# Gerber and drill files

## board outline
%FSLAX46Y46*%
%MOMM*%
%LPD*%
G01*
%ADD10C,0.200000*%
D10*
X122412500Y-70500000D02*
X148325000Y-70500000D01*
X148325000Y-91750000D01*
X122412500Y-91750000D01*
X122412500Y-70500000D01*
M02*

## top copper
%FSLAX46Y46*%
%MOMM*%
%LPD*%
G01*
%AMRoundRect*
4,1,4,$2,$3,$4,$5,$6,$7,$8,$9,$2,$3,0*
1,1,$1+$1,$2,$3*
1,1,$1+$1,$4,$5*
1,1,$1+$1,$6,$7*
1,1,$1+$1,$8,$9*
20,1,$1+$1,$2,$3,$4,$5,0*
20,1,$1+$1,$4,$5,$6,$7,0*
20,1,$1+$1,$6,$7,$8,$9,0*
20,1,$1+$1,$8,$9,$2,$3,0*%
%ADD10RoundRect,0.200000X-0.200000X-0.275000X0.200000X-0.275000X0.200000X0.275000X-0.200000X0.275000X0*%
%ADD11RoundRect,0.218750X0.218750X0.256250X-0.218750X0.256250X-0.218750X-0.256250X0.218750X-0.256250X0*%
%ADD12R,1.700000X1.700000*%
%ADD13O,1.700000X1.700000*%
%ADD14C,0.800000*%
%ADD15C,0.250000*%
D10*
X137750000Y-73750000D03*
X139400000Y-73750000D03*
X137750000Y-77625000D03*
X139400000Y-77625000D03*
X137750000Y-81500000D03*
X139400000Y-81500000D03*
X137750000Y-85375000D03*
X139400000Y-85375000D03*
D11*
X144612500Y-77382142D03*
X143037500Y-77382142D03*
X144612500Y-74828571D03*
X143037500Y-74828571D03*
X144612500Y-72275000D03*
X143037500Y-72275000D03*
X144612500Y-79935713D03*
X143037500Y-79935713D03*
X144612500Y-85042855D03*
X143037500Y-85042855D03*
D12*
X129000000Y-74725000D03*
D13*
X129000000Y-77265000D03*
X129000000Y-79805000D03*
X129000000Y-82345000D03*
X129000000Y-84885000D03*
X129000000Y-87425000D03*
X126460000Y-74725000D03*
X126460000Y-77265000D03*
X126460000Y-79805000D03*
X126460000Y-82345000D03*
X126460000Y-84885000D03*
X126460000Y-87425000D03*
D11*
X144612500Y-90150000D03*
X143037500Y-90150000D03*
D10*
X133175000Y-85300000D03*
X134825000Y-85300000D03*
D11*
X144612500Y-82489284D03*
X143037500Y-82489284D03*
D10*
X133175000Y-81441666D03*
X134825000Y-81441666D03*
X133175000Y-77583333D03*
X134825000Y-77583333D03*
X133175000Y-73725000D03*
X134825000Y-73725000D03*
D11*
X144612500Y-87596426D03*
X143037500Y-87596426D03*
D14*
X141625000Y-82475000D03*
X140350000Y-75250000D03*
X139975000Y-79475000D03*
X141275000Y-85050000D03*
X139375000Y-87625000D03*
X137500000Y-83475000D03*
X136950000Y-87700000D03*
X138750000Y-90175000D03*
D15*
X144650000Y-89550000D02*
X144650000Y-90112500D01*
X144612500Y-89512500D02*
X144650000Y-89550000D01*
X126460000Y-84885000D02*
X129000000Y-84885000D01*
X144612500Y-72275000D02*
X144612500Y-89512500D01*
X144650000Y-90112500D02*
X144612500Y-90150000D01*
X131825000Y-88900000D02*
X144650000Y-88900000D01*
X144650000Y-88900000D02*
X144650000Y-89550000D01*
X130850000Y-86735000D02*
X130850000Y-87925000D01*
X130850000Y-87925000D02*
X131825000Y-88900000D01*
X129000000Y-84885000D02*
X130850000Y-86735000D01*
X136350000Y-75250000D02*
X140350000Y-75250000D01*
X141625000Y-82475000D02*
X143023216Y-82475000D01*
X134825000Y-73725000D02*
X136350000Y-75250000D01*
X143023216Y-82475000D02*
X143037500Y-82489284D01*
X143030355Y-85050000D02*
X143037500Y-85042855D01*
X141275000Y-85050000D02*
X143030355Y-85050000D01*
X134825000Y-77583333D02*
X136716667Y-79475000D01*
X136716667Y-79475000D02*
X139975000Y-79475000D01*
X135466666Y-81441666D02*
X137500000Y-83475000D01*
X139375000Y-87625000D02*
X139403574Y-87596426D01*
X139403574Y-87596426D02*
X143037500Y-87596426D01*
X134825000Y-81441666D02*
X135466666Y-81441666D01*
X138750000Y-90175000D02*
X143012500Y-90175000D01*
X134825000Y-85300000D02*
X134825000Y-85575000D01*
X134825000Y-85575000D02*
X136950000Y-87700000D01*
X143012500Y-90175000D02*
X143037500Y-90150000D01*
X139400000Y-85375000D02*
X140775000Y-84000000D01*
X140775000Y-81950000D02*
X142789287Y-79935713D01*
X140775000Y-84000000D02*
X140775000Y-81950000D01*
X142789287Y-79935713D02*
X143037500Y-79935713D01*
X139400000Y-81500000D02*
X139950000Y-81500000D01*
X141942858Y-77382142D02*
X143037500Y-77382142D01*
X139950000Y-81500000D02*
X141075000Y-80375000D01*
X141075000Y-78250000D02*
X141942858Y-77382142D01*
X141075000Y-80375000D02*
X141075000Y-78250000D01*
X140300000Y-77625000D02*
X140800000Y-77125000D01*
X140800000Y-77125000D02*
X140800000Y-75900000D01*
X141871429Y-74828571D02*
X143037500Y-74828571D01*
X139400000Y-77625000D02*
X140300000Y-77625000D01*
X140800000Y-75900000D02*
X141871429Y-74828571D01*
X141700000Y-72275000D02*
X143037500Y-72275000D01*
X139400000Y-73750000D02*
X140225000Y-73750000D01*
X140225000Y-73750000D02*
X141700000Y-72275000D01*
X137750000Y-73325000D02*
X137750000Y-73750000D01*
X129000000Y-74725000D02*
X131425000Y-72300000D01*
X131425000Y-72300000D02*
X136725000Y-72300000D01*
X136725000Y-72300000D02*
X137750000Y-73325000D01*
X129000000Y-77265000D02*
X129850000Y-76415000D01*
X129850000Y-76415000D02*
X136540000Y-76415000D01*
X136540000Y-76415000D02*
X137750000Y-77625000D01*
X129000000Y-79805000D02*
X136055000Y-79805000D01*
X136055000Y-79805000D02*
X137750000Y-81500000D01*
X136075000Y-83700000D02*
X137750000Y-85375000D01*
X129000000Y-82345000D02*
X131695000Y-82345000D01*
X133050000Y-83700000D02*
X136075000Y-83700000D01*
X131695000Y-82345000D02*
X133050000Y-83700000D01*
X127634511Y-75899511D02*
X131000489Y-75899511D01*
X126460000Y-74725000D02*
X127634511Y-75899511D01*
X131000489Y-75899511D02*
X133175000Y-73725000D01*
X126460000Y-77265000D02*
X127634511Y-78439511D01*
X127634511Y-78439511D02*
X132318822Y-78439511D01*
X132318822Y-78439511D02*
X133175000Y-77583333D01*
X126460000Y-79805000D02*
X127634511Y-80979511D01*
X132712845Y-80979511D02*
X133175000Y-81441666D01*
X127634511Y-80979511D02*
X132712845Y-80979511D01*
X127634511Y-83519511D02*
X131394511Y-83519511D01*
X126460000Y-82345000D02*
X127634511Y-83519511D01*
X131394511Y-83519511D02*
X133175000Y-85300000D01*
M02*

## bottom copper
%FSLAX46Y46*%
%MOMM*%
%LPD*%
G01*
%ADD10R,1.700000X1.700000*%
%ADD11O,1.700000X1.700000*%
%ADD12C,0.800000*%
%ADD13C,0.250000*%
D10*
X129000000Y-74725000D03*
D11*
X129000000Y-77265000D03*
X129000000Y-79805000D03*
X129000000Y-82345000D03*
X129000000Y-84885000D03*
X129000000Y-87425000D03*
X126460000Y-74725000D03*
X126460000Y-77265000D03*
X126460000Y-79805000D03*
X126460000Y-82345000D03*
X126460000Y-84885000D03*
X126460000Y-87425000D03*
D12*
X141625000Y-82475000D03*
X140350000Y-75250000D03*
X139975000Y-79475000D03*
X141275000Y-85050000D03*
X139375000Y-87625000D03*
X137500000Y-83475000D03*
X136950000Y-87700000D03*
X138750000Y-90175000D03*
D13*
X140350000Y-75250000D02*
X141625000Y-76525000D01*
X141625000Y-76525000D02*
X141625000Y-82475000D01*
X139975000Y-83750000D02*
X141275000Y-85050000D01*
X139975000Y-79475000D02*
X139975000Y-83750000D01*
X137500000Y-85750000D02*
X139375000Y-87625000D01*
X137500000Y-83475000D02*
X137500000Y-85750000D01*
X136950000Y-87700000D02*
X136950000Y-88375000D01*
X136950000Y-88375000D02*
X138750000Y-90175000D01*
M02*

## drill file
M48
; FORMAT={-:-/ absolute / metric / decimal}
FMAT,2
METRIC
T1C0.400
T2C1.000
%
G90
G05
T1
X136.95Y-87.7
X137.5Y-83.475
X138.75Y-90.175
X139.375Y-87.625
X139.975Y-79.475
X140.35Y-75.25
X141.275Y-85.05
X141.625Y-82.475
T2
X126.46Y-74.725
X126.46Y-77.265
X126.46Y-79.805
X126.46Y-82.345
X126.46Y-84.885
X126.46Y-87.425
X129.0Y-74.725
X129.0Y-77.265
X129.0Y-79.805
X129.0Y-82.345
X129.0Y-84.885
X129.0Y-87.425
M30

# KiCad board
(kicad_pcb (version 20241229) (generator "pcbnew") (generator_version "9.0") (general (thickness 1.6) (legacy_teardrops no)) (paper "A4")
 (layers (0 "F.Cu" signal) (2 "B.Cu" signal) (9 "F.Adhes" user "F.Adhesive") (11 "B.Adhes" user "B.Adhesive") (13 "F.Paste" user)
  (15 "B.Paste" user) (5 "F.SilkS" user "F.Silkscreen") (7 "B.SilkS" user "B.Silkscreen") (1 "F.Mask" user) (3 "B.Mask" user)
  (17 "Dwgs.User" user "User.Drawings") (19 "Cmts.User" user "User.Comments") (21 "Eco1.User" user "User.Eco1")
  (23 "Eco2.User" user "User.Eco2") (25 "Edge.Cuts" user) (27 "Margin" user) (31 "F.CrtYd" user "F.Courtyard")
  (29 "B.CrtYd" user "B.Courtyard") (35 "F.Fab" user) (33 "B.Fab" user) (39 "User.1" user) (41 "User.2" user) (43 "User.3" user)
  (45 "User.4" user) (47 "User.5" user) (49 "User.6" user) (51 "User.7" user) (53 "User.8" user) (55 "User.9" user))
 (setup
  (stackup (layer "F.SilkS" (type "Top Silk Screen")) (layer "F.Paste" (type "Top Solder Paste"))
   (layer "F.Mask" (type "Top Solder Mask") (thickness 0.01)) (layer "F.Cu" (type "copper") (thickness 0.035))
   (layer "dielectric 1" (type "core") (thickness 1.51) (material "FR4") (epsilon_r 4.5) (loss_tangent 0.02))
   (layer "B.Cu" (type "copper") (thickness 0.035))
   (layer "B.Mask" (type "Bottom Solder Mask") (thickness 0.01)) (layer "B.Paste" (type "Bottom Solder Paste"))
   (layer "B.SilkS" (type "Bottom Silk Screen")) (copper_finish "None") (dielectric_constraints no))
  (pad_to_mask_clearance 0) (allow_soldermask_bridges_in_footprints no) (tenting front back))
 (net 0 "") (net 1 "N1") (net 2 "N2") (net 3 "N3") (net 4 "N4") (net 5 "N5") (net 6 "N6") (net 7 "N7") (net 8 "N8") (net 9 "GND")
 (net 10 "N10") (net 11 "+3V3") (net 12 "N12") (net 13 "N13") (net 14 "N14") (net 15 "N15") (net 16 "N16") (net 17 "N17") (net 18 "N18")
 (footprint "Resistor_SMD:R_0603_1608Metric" (layer "F.Cu") (at 138.575 73.75)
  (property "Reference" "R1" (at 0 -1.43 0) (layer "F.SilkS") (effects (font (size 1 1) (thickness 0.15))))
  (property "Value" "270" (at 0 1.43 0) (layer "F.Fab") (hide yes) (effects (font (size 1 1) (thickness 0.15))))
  (pad "1" smd roundrect (at -0.825 0) (size 0.8 0.95) (layers "F.Cu" "F.Mask" "F.Paste") (roundrect_rratio 0.25) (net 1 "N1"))
  (pad "2" smd roundrect (at 0.825 0) (size 0.8 0.95) (layers "F.Cu" "F.Mask" "F.Paste") (roundrect_rratio 0.25) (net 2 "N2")))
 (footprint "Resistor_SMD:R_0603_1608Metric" (layer "F.Cu") (at 138.575 77.625)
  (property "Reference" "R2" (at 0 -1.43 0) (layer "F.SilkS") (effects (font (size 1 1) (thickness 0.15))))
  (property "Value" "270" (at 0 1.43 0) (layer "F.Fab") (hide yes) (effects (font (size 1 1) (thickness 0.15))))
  (pad "1" smd roundrect (at -0.825 0) (size 0.8 0.95) (layers "F.Cu" "F.Mask" "F.Paste") (roundrect_rratio 0.25) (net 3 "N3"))
  (pad "2" smd roundrect (at 0.825 0) (size 0.8 0.95) (layers "F.Cu" "F.Mask" "F.Paste") (roundrect_rratio 0.25) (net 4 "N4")))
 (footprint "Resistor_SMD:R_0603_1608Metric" (layer "F.Cu") (at 138.575 81.5)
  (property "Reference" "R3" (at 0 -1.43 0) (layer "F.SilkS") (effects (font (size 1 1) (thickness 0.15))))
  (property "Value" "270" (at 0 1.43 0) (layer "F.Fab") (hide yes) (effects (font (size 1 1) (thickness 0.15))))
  (pad "1" smd roundrect (at -0.825 0) (size 0.8 0.95) (layers "F.Cu" "F.Mask" "F.Paste") (roundrect_rratio 0.25) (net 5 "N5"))
  (pad "2" smd roundrect (at 0.825 0) (size 0.8 0.95) (layers "F.Cu" "F.Mask" "F.Paste") (roundrect_rratio 0.25) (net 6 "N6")))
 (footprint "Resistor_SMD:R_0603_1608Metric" (layer "F.Cu") (at 138.575 85.375)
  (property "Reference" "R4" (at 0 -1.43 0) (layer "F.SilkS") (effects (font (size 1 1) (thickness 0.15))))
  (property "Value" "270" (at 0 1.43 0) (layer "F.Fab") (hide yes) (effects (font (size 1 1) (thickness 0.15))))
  (pad "1" smd roundrect (at -0.825 0) (size 0.8 0.95) (layers "F.Cu" "F.Mask" "F.Paste") (roundrect_rratio 0.25) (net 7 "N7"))
  (pad "2" smd roundrect (at 0.825 0) (size 0.8 0.95) (layers "F.Cu" "F.Mask" "F.Paste") (roundrect_rratio 0.25) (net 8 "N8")))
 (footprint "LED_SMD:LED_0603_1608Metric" (layer "F.Cu") (at 143.825 77.382142 180)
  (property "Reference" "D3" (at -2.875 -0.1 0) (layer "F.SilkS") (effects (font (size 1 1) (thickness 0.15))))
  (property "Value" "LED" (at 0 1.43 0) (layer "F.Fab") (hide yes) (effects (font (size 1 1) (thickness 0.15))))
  (pad "1" smd roundrect (at -0.7875 0 180) (size 0.875 0.95) (layers "F.Cu" "F.Mask" "F.Paste") (roundrect_rratio 0.25) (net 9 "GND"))
  (pad "2" smd roundrect (at 0.7875 0 180) (size 0.875 0.95) (layers "F.Cu" "F.Mask" "F.Paste") (roundrect_rratio 0.25) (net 6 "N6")))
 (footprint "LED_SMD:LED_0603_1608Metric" (layer "F.Cu") (at 143.825 74.828571 180)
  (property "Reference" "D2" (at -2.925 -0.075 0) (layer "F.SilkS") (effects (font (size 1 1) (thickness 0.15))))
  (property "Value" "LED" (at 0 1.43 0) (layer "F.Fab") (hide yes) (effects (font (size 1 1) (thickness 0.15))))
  (pad "1" smd roundrect (at -0.7875 0 180) (size 0.875 0.95) (layers "F.Cu" "F.Mask" "F.Paste") (roundrect_rratio 0.25) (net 9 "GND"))
  (pad "2" smd roundrect (at 0.7875 0 180) (size 0.875 0.95) (layers "F.Cu" "F.Mask" "F.Paste") (roundrect_rratio 0.25) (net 4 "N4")))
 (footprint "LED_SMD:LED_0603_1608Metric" (layer "F.Cu") (at 143.825 72.275 180)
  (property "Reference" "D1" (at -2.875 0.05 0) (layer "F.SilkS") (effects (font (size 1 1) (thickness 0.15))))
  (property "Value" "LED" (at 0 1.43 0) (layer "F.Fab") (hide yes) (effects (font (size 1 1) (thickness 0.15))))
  (pad "1" smd roundrect (at -0.7875 0 180) (size 0.875 0.95) (layers "F.Cu" "F.Mask" "F.Paste") (roundrect_rratio 0.25) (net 9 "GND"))
  (pad "2" smd roundrect (at 0.7875 0 180) (size 0.875 0.95) (layers "F.Cu" "F.Mask" "F.Paste") (roundrect_rratio 0.25) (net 2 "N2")))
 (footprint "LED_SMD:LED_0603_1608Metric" (layer "F.Cu") (at 143.825 79.935713 180)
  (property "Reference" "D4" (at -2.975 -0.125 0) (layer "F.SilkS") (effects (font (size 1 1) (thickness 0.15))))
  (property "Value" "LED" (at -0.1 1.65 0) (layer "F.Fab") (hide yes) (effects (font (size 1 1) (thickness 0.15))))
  (pad "1" smd roundrect (at -0.7875 0 180) (size 0.875 0.95) (layers "F.Cu" "F.Mask" "F.Paste") (roundrect_rratio 0.25) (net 9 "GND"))
  (pad "2" smd roundrect (at 0.7875 0 180) (size 0.875 0.95) (layers "F.Cu" "F.Mask" "F.Paste") (roundrect_rratio 0.25) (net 8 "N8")))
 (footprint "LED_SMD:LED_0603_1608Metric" (layer "F.Cu") (at 143.825 85.042855 180)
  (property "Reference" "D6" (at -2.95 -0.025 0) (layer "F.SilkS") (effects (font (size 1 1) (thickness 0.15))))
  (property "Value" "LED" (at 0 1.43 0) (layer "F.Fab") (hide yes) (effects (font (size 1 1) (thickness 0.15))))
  (pad "1" smd roundrect (at -0.7875 0 180) (size 0.875 0.95) (layers "F.Cu" "F.Mask" "F.Paste") (roundrect_rratio 0.25) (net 9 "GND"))
  (pad "2" smd roundrect (at 0.7875 0 180) (size 0.875 0.95) (layers "F.Cu" "F.Mask" "F.Paste") (roundrect_rratio 0.25) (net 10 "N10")))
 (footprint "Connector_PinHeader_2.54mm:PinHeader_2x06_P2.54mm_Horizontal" (layer "F.Cu") (at 129 87.425 180)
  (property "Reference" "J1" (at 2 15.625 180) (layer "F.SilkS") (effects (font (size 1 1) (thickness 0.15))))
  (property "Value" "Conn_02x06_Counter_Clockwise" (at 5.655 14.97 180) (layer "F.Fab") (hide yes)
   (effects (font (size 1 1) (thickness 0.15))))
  (pad "1" thru_hole rect (at 0 12.7 180) (size 1.7 1.7) (drill 1) (layers "*.Cu" "*.Mask") (remove_unused_layers no) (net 1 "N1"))
  (pad "2" thru_hole oval (at 0 10.16 180) (size 1.7 1.7) (drill 1) (layers "*.Cu" "*.Mask") (remove_unused_layers no) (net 3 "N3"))
  (pad "3" thru_hole oval (at 0 7.62 180) (size 1.7 1.7) (drill 1) (layers "*.Cu" "*.Mask") (remove_unused_layers no) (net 5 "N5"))
  (pad "4" thru_hole oval (at 0 5.08 180) (size 1.7 1.7) (drill 1) (layers "*.Cu" "*.Mask") (remove_unused_layers no) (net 7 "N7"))
  (pad "5" thru_hole oval (at 0 2.54 180) (size 1.7 1.7) (drill 1) (layers "*.Cu" "*.Mask") (remove_unused_layers no) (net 9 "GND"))
  (pad "6" thru_hole oval (at 0 0 180) (size 1.7 1.7) (drill 1) (layers "*.Cu" "*.Mask") (remove_unused_layers no) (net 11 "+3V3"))
  (pad "7" thru_hole oval (at 2.54 12.7 180) (size 1.7 1.7) (drill 1) (layers "*.Cu" "*.Mask") (remove_unused_layers no) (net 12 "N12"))
  (pad "8" thru_hole oval (at 2.54 10.16 180) (size 1.7 1.7) (drill 1) (layers "*.Cu" "*.Mask") (remove_unused_layers no) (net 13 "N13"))
  (pad "9" thru_hole oval (at 2.54 7.62 180) (size 1.7 1.7) (drill 1) (layers "*.Cu" "*.Mask") (remove_unused_layers no) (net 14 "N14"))
  (pad "10" thru_hole oval (at 2.54 5.08 180) (size 1.7 1.7) (drill 1) (layers "*.Cu" "*.Mask") (remove_unused_layers no) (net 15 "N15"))
  (pad "11" thru_hole oval (at 2.54 2.54 180) (size 1.7 1.7) (drill 1) (layers "*.Cu" "*.Mask") (remove_unused_layers no) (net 9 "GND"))
  (pad "12" thru_hole oval (at 2.54 0 180) (size 1.7 1.7) (drill 1) (layers "*.Cu" "*.Mask") (remove_unused_layers no) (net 11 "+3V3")))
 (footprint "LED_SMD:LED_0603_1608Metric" (layer "F.Cu") (at 143.825 90.15 180)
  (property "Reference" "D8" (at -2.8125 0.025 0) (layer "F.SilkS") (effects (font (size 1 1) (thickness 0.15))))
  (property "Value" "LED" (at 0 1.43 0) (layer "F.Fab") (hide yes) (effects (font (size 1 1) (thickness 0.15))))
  (pad "1" smd roundrect (at -0.7875 0 180) (size 0.875 0.95) (layers "F.Cu" "F.Mask" "F.Paste") (roundrect_rratio 0.25) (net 9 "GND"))
  (pad "2" smd roundrect (at 0.7875 0 180) (size 0.875 0.95) (layers "F.Cu" "F.Mask" "F.Paste") (roundrect_rratio 0.25) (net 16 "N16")))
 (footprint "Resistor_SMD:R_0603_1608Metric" (layer "F.Cu") (at 134 85.3)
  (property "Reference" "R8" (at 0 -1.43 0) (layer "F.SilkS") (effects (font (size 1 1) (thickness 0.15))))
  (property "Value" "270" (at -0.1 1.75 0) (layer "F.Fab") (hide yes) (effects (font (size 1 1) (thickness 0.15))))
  (pad "1" smd roundrect (at -0.825 0) (size 0.8 0.95) (layers "F.Cu" "F.Mask" "F.Paste") (roundrect_rratio 0.25) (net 15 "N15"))
  (pad "2" smd roundrect (at 0.825 0) (size 0.8 0.95) (layers "F.Cu" "F.Mask" "F.Paste") (roundrect_rratio 0.25) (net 16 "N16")))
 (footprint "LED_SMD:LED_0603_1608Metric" (layer "F.Cu") (at 143.825 82.489284 180)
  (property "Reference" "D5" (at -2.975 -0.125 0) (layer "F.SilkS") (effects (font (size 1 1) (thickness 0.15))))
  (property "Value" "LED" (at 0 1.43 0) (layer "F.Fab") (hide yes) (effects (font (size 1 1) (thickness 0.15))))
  (pad "1" smd roundrect (at -0.7875 0 180) (size 0.875 0.95) (layers "F.Cu" "F.Mask" "F.Paste") (roundrect_rratio 0.25) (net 9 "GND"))
  (pad "2" smd roundrect (at 0.7875 0 180) (size 0.875 0.95) (layers "F.Cu" "F.Mask" "F.Paste") (roundrect_rratio 0.25) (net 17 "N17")))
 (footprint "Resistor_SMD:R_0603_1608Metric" (layer "F.Cu") (at 134 81.441666)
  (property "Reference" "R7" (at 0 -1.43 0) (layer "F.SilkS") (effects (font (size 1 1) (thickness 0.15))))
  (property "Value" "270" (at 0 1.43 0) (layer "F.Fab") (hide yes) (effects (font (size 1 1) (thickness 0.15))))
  (pad "1" smd roundrect (at -0.825 0) (size 0.8 0.95) (layers "F.Cu" "F.Mask" "F.Paste") (roundrect_rratio 0.25) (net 14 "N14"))
  (pad "2" smd roundrect (at 0.825 0) (size 0.8 0.95) (layers "F.Cu" "F.Mask" "F.Paste") (roundrect_rratio 0.25) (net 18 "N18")))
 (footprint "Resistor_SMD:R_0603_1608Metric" (layer "F.Cu") (at 134 77.583333)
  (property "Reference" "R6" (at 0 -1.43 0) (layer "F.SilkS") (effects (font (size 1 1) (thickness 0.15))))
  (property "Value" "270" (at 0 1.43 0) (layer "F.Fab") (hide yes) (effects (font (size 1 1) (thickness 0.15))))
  (pad "1" smd roundrect (at -0.825 0) (size 0.8 0.95) (layers "F.Cu" "F.Mask" "F.Paste") (roundrect_rratio 0.25) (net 13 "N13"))
  (pad "2" smd roundrect (at 0.825 0) (size 0.8 0.95) (layers "F.Cu" "F.Mask" "F.Paste") (roundrect_rratio 0.25) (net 10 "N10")))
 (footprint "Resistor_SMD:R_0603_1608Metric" (layer "F.Cu") (at 134 73.725)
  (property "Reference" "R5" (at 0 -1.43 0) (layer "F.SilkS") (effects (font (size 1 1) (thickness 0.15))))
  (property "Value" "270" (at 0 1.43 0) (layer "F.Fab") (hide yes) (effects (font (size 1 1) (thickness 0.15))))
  (pad "1" smd roundrect (at -0.825 0) (size 0.8 0.95) (layers "F.Cu" "F.Mask" "F.Paste") (roundrect_rratio 0.25) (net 12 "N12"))
  (pad "2" smd roundrect (at 0.825 0) (size 0.8 0.95) (layers "F.Cu" "F.Mask" "F.Paste") (roundrect_rratio 0.25) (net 17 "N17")))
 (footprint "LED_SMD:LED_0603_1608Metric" (layer "F.Cu") (at 143.825 87.596426 180)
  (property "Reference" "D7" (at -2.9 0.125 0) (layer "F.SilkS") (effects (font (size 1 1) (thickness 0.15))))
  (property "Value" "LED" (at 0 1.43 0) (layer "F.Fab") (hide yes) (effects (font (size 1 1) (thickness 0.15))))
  (pad "1" smd roundrect (at -0.7875 0 180) (size 0.875 0.95) (layers "F.Cu" "F.Mask" "F.Paste") (roundrect_rratio 0.25) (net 9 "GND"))
  (pad "2" smd roundrect (at 0.7875 0 180) (size 0.875 0.95) (layers "F.Cu" "F.Mask" "F.Paste") (roundrect_rratio 0.25) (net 18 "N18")))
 (gr_rect (start 122.4125 70.5) (end 148.325 91.75) (stroke (width 0.2) (type solid)) (fill no) (layer "Edge.Cuts"))
 (segment (start 144.65 89.55) (end 144.65 90.1125) (width 0.25) (layer "F.Cu") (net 9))
 (segment (start 144.6125 89.5125) (end 144.65 89.55) (width 0.25) (layer "F.Cu") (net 9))
 (segment (start 126.46 84.885) (end 129 84.885) (width 0.25) (layer "F.Cu") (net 9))
 (segment (start 144.6125 72.275) (end 144.6125 89.5125) (width 0.25) (layer "F.Cu") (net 9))
 (segment (start 144.65 90.1125) (end 144.6125 90.15) (width 0.25) (layer "F.Cu") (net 9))
 (segment (start 131.825 88.9) (end 144.65 88.9) (width 0.25) (layer "F.Cu") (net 9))
 (segment (start 144.65 88.9) (end 144.65 89.55) (width 0.25) (layer "F.Cu") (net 9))
 (segment (start 130.85 86.735) (end 130.85 87.925) (width 0.25) (layer "F.Cu") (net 9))
 (segment (start 130.85 87.925) (end 131.825 88.9) (width 0.25) (layer "F.Cu") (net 9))
 (segment (start 129 84.885) (end 130.85 86.735) (width 0.25) (layer "F.Cu") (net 9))
 (segment (start 136.35 75.25) (end 140.35 75.25) (width 0.25) (layer "F.Cu") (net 17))
 (segment (start 141.625 82.475) (end 143.023216 82.475) (width 0.25) (layer "F.Cu") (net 17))
 (segment (start 134.825 73.725) (end 136.35 75.25) (width 0.25) (layer "F.Cu") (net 17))
 (segment (start 143.023216 82.475) (end 143.0375 82.489284) (width 0.25) (layer "F.Cu") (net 17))
 (via (at 141.625 82.475) (size 0.8) (drill 0.4) (layers "F.Cu" "B.Cu") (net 17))
 (via (at 140.35 75.25) (size 0.8) (drill 0.4) (layers "F.Cu" "B.Cu") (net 17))
 (segment (start 140.35 75.25) (end 141.625 76.525) (width 0.25) (layer "B.Cu") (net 17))
 (segment (start 141.625 76.525) (end 141.625 82.475) (width 0.25) (layer "B.Cu") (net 17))
 (segment (start 143.030355 85.05) (end 143.0375 85.042855) (width 0.25) (layer "F.Cu") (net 10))
 (segment (start 141.275 85.05) (end 143.030355 85.05) (width 0.25) (layer "F.Cu") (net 10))
 (segment (start 134.825 77.583333) (end 136.716667 79.475) (width 0.25) (layer "F.Cu") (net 10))
 (segment (start 136.716667 79.475) (end 139.975 79.475) (width 0.25) (layer "F.Cu") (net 10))
 (via (at 139.975 79.475) (size 0.8) (drill 0.4) (layers "F.Cu" "B.Cu") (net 10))
 (via (at 141.275 85.05) (size 0.8) (drill 0.4) (layers "F.Cu" "B.Cu") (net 10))
 (segment (start 139.975 83.75) (end 141.275 85.05) (width 0.25) (layer "B.Cu") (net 10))
 (segment (start 139.975 79.475) (end 139.975 83.75) (width 0.25) (layer "B.Cu") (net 10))
 (segment (start 135.466666 81.441666) (end 137.5 83.475) (width 0.25) (layer "F.Cu") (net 18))
 (segment (start 139.375 87.625) (end 139.403574 87.596426) (width 0.25) (layer "F.Cu") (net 18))
 (segment (start 139.403574 87.596426) (end 143.0375 87.596426) (width 0.25) (layer "F.Cu") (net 18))
 (segment (start 134.825 81.441666) (end 135.466666 81.441666) (width 0.25) (layer "F.Cu") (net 18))
 (via (at 139.375 87.625) (size 0.8) (drill 0.4) (layers "F.Cu" "B.Cu") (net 18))
 (via (at 137.5 83.475) (size 0.8) (drill 0.4) (layers "F.Cu" "B.Cu") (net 18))
 (segment (start 137.5 85.75) (end 139.375 87.625) (width 0.25) (layer "B.Cu") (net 18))
 (segment (start 137.5 83.475) (end 137.5 85.75) (width 0.25) (layer "B.Cu") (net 18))
 (segment (start 138.75 90.175) (end 143.0125 90.175) (width 0.25) (layer "F.Cu") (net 16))
 (segment (start 134.825 85.3) (end 134.825 85.575) (width 0.25) (layer "F.Cu") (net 16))
 (segment (start 134.825 85.575) (end 136.95 87.7) (width 0.25) (layer "F.Cu") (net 16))
 (segment (start 143.0125 90.175) (end 143.0375 90.15) (width 0.25) (layer "F.Cu") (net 16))
 (via (at 136.95 87.7) (size 0.8) (drill 0.4) (layers "F.Cu" "B.Cu") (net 16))
 (via (at 138.75 90.175) (size 0.8) (drill 0.4) (layers "F.Cu" "B.Cu") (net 16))
 (segment (start 136.95 87.7) (end 136.95 88.375) (width 0.25) (layer "B.Cu") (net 16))
 (segment (start 136.95 88.375) (end 138.75 90.175) (width 0.25) (layer "B.Cu") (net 16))
 (segment (start 139.4 85.375) (end 140.775 84) (width 0.25) (layer "F.Cu") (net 8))
 (segment (start 140.775 81.95) (end 142.789287 79.935713) (width 0.25) (layer "F.Cu") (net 8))
 (segment (start 140.775 84) (end 140.775 81.95) (width 0.25) (layer "F.Cu") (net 8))
 (segment (start 142.789287 79.935713) (end 143.0375 79.935713) (width 0.25) (layer "F.Cu") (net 8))
 (segment (start 139.4 81.5) (end 139.95 81.5) (width 0.25) (layer "F.Cu") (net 6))
 (segment (start 141.942858 77.382142) (end 143.0375 77.382142) (width 0.25) (layer "F.Cu") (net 6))
 (segment (start 139.95 81.5) (end 141.075 80.375) (width 0.25) (layer "F.Cu") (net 6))
 (segment (start 141.075 78.25) (end 141.942858 77.382142) (width 0.25) (layer "F.Cu") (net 6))
 (segment (start 141.075 80.375) (end 141.075 78.25) (width 0.25) (layer "F.Cu") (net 6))
 (segment (start 140.3 77.625) (end 140.8 77.125) (width 0.25) (layer "F.Cu") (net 4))
 (segment (start 140.8 77.125) (end 140.8 75.9) (width 0.25) (layer "F.Cu") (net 4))
 (segment (start 141.871429 74.828571) (end 143.0375 74.828571) (width 0.25) (layer "F.Cu") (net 4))
 (segment (start 139.4 77.625) (end 140.3 77.625) (width 0.25) (layer "F.Cu") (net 4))
 (segment (start 140.8 75.9) (end 141.871429 74.828571) (width 0.25) (layer "F.Cu") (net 4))
 (segment (start 141.7 72.275) (end 143.0375 72.275) (width 0.25) (layer "F.Cu") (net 2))
 (segment (start 139.4 73.75) (end 140.225 73.75) (width 0.25) (layer "F.Cu") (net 2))
 (segment (start 140.225 73.75) (end 141.7 72.275) (width 0.25) (layer "F.Cu") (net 2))
 (segment (start 137.75 73.325) (end 137.75 73.75) (width 0.25) (layer "F.Cu") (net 1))
 (segment (start 129 74.725) (end 131.425 72.3) (width 0.25) (layer "F.Cu") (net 1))
 (segment (start 131.425 72.3) (end 136.725 72.3) (width 0.25) (layer "F.Cu") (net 1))
 (segment (start 136.725 72.3) (end 137.75 73.325) (width 0.25) (layer "F.Cu") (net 1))
 (segment (start 129 77.265) (end 129.85 76.415) (width 0.25) (layer "F.Cu") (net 3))
 (segment (start 129.85 76.415) (end 136.54 76.415) (width 0.25) (layer "F.Cu") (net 3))
 (segment (start 136.54 76.415) (end 137.75 77.625) (width 0.25) (layer "F.Cu") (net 3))
 (segment (start 129 79.805) (end 136.055 79.805) (width 0.25) (layer "F.Cu") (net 5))
 (segment (start 136.055 79.805) (end 137.75 81.5) (width 0.25) (layer "F.Cu") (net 5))
 (segment (start 136.075 83.7) (end 137.75 85.375) (width 0.25) (layer "F.Cu") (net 7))
 (segment (start 129 82.345) (end 131.695 82.345) (width 0.25) (layer "F.Cu") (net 7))
 (segment (start 133.05 83.7) (end 136.075 83.7) (width 0.25) (layer "F.Cu") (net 7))
 (segment (start 131.695 82.345) (end 133.05 83.7) (width 0.25) (layer "F.Cu") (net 7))
 (segment (start 127.634511 75.899511) (end 131.000489 75.899511) (width 0.25) (layer "F.Cu") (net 12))
 (segment (start 126.46 74.725) (end 127.634511 75.899511) (width 0.25) (layer "F.Cu") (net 12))
 (segment (start 131.000489 75.899511) (end 133.175 73.725) (width 0.25) (layer "F.Cu") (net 12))
 (segment (start 126.46 77.265) (end 127.634511 78.439511) (width 0.25) (layer "F.Cu") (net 13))
 (segment (start 127.634511 78.439511) (end 132.318822 78.439511) (width 0.25) (layer "F.Cu") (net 13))
 (segment (start 132.318822 78.439511) (end 133.175 77.583333) (width 0.25) (layer "F.Cu") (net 13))
 (segment (start 126.46 79.805) (end 127.634511 80.979511) (width 0.25) (layer "F.Cu") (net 14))
 (segment (start 132.712845 80.979511) (end 133.175 81.441666) (width 0.25) (layer "F.Cu") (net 14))
 (segment (start 127.634511 80.979511) (end 132.712845 80.979511) (width 0.25) (layer "F.Cu") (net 14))
 (segment (start 127.634511 83.519511) (end 131.394511 83.519511) (width 0.25) (layer "F.Cu") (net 15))
 (segment (start 126.46 82.345) (end 127.634511 83.519511) (width 0.25) (layer "F.Cu") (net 15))
 (segment (start 131.394511 83.519511) (end 133.175 85.3) (width 0.25) (layer "F.Cu") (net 15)))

